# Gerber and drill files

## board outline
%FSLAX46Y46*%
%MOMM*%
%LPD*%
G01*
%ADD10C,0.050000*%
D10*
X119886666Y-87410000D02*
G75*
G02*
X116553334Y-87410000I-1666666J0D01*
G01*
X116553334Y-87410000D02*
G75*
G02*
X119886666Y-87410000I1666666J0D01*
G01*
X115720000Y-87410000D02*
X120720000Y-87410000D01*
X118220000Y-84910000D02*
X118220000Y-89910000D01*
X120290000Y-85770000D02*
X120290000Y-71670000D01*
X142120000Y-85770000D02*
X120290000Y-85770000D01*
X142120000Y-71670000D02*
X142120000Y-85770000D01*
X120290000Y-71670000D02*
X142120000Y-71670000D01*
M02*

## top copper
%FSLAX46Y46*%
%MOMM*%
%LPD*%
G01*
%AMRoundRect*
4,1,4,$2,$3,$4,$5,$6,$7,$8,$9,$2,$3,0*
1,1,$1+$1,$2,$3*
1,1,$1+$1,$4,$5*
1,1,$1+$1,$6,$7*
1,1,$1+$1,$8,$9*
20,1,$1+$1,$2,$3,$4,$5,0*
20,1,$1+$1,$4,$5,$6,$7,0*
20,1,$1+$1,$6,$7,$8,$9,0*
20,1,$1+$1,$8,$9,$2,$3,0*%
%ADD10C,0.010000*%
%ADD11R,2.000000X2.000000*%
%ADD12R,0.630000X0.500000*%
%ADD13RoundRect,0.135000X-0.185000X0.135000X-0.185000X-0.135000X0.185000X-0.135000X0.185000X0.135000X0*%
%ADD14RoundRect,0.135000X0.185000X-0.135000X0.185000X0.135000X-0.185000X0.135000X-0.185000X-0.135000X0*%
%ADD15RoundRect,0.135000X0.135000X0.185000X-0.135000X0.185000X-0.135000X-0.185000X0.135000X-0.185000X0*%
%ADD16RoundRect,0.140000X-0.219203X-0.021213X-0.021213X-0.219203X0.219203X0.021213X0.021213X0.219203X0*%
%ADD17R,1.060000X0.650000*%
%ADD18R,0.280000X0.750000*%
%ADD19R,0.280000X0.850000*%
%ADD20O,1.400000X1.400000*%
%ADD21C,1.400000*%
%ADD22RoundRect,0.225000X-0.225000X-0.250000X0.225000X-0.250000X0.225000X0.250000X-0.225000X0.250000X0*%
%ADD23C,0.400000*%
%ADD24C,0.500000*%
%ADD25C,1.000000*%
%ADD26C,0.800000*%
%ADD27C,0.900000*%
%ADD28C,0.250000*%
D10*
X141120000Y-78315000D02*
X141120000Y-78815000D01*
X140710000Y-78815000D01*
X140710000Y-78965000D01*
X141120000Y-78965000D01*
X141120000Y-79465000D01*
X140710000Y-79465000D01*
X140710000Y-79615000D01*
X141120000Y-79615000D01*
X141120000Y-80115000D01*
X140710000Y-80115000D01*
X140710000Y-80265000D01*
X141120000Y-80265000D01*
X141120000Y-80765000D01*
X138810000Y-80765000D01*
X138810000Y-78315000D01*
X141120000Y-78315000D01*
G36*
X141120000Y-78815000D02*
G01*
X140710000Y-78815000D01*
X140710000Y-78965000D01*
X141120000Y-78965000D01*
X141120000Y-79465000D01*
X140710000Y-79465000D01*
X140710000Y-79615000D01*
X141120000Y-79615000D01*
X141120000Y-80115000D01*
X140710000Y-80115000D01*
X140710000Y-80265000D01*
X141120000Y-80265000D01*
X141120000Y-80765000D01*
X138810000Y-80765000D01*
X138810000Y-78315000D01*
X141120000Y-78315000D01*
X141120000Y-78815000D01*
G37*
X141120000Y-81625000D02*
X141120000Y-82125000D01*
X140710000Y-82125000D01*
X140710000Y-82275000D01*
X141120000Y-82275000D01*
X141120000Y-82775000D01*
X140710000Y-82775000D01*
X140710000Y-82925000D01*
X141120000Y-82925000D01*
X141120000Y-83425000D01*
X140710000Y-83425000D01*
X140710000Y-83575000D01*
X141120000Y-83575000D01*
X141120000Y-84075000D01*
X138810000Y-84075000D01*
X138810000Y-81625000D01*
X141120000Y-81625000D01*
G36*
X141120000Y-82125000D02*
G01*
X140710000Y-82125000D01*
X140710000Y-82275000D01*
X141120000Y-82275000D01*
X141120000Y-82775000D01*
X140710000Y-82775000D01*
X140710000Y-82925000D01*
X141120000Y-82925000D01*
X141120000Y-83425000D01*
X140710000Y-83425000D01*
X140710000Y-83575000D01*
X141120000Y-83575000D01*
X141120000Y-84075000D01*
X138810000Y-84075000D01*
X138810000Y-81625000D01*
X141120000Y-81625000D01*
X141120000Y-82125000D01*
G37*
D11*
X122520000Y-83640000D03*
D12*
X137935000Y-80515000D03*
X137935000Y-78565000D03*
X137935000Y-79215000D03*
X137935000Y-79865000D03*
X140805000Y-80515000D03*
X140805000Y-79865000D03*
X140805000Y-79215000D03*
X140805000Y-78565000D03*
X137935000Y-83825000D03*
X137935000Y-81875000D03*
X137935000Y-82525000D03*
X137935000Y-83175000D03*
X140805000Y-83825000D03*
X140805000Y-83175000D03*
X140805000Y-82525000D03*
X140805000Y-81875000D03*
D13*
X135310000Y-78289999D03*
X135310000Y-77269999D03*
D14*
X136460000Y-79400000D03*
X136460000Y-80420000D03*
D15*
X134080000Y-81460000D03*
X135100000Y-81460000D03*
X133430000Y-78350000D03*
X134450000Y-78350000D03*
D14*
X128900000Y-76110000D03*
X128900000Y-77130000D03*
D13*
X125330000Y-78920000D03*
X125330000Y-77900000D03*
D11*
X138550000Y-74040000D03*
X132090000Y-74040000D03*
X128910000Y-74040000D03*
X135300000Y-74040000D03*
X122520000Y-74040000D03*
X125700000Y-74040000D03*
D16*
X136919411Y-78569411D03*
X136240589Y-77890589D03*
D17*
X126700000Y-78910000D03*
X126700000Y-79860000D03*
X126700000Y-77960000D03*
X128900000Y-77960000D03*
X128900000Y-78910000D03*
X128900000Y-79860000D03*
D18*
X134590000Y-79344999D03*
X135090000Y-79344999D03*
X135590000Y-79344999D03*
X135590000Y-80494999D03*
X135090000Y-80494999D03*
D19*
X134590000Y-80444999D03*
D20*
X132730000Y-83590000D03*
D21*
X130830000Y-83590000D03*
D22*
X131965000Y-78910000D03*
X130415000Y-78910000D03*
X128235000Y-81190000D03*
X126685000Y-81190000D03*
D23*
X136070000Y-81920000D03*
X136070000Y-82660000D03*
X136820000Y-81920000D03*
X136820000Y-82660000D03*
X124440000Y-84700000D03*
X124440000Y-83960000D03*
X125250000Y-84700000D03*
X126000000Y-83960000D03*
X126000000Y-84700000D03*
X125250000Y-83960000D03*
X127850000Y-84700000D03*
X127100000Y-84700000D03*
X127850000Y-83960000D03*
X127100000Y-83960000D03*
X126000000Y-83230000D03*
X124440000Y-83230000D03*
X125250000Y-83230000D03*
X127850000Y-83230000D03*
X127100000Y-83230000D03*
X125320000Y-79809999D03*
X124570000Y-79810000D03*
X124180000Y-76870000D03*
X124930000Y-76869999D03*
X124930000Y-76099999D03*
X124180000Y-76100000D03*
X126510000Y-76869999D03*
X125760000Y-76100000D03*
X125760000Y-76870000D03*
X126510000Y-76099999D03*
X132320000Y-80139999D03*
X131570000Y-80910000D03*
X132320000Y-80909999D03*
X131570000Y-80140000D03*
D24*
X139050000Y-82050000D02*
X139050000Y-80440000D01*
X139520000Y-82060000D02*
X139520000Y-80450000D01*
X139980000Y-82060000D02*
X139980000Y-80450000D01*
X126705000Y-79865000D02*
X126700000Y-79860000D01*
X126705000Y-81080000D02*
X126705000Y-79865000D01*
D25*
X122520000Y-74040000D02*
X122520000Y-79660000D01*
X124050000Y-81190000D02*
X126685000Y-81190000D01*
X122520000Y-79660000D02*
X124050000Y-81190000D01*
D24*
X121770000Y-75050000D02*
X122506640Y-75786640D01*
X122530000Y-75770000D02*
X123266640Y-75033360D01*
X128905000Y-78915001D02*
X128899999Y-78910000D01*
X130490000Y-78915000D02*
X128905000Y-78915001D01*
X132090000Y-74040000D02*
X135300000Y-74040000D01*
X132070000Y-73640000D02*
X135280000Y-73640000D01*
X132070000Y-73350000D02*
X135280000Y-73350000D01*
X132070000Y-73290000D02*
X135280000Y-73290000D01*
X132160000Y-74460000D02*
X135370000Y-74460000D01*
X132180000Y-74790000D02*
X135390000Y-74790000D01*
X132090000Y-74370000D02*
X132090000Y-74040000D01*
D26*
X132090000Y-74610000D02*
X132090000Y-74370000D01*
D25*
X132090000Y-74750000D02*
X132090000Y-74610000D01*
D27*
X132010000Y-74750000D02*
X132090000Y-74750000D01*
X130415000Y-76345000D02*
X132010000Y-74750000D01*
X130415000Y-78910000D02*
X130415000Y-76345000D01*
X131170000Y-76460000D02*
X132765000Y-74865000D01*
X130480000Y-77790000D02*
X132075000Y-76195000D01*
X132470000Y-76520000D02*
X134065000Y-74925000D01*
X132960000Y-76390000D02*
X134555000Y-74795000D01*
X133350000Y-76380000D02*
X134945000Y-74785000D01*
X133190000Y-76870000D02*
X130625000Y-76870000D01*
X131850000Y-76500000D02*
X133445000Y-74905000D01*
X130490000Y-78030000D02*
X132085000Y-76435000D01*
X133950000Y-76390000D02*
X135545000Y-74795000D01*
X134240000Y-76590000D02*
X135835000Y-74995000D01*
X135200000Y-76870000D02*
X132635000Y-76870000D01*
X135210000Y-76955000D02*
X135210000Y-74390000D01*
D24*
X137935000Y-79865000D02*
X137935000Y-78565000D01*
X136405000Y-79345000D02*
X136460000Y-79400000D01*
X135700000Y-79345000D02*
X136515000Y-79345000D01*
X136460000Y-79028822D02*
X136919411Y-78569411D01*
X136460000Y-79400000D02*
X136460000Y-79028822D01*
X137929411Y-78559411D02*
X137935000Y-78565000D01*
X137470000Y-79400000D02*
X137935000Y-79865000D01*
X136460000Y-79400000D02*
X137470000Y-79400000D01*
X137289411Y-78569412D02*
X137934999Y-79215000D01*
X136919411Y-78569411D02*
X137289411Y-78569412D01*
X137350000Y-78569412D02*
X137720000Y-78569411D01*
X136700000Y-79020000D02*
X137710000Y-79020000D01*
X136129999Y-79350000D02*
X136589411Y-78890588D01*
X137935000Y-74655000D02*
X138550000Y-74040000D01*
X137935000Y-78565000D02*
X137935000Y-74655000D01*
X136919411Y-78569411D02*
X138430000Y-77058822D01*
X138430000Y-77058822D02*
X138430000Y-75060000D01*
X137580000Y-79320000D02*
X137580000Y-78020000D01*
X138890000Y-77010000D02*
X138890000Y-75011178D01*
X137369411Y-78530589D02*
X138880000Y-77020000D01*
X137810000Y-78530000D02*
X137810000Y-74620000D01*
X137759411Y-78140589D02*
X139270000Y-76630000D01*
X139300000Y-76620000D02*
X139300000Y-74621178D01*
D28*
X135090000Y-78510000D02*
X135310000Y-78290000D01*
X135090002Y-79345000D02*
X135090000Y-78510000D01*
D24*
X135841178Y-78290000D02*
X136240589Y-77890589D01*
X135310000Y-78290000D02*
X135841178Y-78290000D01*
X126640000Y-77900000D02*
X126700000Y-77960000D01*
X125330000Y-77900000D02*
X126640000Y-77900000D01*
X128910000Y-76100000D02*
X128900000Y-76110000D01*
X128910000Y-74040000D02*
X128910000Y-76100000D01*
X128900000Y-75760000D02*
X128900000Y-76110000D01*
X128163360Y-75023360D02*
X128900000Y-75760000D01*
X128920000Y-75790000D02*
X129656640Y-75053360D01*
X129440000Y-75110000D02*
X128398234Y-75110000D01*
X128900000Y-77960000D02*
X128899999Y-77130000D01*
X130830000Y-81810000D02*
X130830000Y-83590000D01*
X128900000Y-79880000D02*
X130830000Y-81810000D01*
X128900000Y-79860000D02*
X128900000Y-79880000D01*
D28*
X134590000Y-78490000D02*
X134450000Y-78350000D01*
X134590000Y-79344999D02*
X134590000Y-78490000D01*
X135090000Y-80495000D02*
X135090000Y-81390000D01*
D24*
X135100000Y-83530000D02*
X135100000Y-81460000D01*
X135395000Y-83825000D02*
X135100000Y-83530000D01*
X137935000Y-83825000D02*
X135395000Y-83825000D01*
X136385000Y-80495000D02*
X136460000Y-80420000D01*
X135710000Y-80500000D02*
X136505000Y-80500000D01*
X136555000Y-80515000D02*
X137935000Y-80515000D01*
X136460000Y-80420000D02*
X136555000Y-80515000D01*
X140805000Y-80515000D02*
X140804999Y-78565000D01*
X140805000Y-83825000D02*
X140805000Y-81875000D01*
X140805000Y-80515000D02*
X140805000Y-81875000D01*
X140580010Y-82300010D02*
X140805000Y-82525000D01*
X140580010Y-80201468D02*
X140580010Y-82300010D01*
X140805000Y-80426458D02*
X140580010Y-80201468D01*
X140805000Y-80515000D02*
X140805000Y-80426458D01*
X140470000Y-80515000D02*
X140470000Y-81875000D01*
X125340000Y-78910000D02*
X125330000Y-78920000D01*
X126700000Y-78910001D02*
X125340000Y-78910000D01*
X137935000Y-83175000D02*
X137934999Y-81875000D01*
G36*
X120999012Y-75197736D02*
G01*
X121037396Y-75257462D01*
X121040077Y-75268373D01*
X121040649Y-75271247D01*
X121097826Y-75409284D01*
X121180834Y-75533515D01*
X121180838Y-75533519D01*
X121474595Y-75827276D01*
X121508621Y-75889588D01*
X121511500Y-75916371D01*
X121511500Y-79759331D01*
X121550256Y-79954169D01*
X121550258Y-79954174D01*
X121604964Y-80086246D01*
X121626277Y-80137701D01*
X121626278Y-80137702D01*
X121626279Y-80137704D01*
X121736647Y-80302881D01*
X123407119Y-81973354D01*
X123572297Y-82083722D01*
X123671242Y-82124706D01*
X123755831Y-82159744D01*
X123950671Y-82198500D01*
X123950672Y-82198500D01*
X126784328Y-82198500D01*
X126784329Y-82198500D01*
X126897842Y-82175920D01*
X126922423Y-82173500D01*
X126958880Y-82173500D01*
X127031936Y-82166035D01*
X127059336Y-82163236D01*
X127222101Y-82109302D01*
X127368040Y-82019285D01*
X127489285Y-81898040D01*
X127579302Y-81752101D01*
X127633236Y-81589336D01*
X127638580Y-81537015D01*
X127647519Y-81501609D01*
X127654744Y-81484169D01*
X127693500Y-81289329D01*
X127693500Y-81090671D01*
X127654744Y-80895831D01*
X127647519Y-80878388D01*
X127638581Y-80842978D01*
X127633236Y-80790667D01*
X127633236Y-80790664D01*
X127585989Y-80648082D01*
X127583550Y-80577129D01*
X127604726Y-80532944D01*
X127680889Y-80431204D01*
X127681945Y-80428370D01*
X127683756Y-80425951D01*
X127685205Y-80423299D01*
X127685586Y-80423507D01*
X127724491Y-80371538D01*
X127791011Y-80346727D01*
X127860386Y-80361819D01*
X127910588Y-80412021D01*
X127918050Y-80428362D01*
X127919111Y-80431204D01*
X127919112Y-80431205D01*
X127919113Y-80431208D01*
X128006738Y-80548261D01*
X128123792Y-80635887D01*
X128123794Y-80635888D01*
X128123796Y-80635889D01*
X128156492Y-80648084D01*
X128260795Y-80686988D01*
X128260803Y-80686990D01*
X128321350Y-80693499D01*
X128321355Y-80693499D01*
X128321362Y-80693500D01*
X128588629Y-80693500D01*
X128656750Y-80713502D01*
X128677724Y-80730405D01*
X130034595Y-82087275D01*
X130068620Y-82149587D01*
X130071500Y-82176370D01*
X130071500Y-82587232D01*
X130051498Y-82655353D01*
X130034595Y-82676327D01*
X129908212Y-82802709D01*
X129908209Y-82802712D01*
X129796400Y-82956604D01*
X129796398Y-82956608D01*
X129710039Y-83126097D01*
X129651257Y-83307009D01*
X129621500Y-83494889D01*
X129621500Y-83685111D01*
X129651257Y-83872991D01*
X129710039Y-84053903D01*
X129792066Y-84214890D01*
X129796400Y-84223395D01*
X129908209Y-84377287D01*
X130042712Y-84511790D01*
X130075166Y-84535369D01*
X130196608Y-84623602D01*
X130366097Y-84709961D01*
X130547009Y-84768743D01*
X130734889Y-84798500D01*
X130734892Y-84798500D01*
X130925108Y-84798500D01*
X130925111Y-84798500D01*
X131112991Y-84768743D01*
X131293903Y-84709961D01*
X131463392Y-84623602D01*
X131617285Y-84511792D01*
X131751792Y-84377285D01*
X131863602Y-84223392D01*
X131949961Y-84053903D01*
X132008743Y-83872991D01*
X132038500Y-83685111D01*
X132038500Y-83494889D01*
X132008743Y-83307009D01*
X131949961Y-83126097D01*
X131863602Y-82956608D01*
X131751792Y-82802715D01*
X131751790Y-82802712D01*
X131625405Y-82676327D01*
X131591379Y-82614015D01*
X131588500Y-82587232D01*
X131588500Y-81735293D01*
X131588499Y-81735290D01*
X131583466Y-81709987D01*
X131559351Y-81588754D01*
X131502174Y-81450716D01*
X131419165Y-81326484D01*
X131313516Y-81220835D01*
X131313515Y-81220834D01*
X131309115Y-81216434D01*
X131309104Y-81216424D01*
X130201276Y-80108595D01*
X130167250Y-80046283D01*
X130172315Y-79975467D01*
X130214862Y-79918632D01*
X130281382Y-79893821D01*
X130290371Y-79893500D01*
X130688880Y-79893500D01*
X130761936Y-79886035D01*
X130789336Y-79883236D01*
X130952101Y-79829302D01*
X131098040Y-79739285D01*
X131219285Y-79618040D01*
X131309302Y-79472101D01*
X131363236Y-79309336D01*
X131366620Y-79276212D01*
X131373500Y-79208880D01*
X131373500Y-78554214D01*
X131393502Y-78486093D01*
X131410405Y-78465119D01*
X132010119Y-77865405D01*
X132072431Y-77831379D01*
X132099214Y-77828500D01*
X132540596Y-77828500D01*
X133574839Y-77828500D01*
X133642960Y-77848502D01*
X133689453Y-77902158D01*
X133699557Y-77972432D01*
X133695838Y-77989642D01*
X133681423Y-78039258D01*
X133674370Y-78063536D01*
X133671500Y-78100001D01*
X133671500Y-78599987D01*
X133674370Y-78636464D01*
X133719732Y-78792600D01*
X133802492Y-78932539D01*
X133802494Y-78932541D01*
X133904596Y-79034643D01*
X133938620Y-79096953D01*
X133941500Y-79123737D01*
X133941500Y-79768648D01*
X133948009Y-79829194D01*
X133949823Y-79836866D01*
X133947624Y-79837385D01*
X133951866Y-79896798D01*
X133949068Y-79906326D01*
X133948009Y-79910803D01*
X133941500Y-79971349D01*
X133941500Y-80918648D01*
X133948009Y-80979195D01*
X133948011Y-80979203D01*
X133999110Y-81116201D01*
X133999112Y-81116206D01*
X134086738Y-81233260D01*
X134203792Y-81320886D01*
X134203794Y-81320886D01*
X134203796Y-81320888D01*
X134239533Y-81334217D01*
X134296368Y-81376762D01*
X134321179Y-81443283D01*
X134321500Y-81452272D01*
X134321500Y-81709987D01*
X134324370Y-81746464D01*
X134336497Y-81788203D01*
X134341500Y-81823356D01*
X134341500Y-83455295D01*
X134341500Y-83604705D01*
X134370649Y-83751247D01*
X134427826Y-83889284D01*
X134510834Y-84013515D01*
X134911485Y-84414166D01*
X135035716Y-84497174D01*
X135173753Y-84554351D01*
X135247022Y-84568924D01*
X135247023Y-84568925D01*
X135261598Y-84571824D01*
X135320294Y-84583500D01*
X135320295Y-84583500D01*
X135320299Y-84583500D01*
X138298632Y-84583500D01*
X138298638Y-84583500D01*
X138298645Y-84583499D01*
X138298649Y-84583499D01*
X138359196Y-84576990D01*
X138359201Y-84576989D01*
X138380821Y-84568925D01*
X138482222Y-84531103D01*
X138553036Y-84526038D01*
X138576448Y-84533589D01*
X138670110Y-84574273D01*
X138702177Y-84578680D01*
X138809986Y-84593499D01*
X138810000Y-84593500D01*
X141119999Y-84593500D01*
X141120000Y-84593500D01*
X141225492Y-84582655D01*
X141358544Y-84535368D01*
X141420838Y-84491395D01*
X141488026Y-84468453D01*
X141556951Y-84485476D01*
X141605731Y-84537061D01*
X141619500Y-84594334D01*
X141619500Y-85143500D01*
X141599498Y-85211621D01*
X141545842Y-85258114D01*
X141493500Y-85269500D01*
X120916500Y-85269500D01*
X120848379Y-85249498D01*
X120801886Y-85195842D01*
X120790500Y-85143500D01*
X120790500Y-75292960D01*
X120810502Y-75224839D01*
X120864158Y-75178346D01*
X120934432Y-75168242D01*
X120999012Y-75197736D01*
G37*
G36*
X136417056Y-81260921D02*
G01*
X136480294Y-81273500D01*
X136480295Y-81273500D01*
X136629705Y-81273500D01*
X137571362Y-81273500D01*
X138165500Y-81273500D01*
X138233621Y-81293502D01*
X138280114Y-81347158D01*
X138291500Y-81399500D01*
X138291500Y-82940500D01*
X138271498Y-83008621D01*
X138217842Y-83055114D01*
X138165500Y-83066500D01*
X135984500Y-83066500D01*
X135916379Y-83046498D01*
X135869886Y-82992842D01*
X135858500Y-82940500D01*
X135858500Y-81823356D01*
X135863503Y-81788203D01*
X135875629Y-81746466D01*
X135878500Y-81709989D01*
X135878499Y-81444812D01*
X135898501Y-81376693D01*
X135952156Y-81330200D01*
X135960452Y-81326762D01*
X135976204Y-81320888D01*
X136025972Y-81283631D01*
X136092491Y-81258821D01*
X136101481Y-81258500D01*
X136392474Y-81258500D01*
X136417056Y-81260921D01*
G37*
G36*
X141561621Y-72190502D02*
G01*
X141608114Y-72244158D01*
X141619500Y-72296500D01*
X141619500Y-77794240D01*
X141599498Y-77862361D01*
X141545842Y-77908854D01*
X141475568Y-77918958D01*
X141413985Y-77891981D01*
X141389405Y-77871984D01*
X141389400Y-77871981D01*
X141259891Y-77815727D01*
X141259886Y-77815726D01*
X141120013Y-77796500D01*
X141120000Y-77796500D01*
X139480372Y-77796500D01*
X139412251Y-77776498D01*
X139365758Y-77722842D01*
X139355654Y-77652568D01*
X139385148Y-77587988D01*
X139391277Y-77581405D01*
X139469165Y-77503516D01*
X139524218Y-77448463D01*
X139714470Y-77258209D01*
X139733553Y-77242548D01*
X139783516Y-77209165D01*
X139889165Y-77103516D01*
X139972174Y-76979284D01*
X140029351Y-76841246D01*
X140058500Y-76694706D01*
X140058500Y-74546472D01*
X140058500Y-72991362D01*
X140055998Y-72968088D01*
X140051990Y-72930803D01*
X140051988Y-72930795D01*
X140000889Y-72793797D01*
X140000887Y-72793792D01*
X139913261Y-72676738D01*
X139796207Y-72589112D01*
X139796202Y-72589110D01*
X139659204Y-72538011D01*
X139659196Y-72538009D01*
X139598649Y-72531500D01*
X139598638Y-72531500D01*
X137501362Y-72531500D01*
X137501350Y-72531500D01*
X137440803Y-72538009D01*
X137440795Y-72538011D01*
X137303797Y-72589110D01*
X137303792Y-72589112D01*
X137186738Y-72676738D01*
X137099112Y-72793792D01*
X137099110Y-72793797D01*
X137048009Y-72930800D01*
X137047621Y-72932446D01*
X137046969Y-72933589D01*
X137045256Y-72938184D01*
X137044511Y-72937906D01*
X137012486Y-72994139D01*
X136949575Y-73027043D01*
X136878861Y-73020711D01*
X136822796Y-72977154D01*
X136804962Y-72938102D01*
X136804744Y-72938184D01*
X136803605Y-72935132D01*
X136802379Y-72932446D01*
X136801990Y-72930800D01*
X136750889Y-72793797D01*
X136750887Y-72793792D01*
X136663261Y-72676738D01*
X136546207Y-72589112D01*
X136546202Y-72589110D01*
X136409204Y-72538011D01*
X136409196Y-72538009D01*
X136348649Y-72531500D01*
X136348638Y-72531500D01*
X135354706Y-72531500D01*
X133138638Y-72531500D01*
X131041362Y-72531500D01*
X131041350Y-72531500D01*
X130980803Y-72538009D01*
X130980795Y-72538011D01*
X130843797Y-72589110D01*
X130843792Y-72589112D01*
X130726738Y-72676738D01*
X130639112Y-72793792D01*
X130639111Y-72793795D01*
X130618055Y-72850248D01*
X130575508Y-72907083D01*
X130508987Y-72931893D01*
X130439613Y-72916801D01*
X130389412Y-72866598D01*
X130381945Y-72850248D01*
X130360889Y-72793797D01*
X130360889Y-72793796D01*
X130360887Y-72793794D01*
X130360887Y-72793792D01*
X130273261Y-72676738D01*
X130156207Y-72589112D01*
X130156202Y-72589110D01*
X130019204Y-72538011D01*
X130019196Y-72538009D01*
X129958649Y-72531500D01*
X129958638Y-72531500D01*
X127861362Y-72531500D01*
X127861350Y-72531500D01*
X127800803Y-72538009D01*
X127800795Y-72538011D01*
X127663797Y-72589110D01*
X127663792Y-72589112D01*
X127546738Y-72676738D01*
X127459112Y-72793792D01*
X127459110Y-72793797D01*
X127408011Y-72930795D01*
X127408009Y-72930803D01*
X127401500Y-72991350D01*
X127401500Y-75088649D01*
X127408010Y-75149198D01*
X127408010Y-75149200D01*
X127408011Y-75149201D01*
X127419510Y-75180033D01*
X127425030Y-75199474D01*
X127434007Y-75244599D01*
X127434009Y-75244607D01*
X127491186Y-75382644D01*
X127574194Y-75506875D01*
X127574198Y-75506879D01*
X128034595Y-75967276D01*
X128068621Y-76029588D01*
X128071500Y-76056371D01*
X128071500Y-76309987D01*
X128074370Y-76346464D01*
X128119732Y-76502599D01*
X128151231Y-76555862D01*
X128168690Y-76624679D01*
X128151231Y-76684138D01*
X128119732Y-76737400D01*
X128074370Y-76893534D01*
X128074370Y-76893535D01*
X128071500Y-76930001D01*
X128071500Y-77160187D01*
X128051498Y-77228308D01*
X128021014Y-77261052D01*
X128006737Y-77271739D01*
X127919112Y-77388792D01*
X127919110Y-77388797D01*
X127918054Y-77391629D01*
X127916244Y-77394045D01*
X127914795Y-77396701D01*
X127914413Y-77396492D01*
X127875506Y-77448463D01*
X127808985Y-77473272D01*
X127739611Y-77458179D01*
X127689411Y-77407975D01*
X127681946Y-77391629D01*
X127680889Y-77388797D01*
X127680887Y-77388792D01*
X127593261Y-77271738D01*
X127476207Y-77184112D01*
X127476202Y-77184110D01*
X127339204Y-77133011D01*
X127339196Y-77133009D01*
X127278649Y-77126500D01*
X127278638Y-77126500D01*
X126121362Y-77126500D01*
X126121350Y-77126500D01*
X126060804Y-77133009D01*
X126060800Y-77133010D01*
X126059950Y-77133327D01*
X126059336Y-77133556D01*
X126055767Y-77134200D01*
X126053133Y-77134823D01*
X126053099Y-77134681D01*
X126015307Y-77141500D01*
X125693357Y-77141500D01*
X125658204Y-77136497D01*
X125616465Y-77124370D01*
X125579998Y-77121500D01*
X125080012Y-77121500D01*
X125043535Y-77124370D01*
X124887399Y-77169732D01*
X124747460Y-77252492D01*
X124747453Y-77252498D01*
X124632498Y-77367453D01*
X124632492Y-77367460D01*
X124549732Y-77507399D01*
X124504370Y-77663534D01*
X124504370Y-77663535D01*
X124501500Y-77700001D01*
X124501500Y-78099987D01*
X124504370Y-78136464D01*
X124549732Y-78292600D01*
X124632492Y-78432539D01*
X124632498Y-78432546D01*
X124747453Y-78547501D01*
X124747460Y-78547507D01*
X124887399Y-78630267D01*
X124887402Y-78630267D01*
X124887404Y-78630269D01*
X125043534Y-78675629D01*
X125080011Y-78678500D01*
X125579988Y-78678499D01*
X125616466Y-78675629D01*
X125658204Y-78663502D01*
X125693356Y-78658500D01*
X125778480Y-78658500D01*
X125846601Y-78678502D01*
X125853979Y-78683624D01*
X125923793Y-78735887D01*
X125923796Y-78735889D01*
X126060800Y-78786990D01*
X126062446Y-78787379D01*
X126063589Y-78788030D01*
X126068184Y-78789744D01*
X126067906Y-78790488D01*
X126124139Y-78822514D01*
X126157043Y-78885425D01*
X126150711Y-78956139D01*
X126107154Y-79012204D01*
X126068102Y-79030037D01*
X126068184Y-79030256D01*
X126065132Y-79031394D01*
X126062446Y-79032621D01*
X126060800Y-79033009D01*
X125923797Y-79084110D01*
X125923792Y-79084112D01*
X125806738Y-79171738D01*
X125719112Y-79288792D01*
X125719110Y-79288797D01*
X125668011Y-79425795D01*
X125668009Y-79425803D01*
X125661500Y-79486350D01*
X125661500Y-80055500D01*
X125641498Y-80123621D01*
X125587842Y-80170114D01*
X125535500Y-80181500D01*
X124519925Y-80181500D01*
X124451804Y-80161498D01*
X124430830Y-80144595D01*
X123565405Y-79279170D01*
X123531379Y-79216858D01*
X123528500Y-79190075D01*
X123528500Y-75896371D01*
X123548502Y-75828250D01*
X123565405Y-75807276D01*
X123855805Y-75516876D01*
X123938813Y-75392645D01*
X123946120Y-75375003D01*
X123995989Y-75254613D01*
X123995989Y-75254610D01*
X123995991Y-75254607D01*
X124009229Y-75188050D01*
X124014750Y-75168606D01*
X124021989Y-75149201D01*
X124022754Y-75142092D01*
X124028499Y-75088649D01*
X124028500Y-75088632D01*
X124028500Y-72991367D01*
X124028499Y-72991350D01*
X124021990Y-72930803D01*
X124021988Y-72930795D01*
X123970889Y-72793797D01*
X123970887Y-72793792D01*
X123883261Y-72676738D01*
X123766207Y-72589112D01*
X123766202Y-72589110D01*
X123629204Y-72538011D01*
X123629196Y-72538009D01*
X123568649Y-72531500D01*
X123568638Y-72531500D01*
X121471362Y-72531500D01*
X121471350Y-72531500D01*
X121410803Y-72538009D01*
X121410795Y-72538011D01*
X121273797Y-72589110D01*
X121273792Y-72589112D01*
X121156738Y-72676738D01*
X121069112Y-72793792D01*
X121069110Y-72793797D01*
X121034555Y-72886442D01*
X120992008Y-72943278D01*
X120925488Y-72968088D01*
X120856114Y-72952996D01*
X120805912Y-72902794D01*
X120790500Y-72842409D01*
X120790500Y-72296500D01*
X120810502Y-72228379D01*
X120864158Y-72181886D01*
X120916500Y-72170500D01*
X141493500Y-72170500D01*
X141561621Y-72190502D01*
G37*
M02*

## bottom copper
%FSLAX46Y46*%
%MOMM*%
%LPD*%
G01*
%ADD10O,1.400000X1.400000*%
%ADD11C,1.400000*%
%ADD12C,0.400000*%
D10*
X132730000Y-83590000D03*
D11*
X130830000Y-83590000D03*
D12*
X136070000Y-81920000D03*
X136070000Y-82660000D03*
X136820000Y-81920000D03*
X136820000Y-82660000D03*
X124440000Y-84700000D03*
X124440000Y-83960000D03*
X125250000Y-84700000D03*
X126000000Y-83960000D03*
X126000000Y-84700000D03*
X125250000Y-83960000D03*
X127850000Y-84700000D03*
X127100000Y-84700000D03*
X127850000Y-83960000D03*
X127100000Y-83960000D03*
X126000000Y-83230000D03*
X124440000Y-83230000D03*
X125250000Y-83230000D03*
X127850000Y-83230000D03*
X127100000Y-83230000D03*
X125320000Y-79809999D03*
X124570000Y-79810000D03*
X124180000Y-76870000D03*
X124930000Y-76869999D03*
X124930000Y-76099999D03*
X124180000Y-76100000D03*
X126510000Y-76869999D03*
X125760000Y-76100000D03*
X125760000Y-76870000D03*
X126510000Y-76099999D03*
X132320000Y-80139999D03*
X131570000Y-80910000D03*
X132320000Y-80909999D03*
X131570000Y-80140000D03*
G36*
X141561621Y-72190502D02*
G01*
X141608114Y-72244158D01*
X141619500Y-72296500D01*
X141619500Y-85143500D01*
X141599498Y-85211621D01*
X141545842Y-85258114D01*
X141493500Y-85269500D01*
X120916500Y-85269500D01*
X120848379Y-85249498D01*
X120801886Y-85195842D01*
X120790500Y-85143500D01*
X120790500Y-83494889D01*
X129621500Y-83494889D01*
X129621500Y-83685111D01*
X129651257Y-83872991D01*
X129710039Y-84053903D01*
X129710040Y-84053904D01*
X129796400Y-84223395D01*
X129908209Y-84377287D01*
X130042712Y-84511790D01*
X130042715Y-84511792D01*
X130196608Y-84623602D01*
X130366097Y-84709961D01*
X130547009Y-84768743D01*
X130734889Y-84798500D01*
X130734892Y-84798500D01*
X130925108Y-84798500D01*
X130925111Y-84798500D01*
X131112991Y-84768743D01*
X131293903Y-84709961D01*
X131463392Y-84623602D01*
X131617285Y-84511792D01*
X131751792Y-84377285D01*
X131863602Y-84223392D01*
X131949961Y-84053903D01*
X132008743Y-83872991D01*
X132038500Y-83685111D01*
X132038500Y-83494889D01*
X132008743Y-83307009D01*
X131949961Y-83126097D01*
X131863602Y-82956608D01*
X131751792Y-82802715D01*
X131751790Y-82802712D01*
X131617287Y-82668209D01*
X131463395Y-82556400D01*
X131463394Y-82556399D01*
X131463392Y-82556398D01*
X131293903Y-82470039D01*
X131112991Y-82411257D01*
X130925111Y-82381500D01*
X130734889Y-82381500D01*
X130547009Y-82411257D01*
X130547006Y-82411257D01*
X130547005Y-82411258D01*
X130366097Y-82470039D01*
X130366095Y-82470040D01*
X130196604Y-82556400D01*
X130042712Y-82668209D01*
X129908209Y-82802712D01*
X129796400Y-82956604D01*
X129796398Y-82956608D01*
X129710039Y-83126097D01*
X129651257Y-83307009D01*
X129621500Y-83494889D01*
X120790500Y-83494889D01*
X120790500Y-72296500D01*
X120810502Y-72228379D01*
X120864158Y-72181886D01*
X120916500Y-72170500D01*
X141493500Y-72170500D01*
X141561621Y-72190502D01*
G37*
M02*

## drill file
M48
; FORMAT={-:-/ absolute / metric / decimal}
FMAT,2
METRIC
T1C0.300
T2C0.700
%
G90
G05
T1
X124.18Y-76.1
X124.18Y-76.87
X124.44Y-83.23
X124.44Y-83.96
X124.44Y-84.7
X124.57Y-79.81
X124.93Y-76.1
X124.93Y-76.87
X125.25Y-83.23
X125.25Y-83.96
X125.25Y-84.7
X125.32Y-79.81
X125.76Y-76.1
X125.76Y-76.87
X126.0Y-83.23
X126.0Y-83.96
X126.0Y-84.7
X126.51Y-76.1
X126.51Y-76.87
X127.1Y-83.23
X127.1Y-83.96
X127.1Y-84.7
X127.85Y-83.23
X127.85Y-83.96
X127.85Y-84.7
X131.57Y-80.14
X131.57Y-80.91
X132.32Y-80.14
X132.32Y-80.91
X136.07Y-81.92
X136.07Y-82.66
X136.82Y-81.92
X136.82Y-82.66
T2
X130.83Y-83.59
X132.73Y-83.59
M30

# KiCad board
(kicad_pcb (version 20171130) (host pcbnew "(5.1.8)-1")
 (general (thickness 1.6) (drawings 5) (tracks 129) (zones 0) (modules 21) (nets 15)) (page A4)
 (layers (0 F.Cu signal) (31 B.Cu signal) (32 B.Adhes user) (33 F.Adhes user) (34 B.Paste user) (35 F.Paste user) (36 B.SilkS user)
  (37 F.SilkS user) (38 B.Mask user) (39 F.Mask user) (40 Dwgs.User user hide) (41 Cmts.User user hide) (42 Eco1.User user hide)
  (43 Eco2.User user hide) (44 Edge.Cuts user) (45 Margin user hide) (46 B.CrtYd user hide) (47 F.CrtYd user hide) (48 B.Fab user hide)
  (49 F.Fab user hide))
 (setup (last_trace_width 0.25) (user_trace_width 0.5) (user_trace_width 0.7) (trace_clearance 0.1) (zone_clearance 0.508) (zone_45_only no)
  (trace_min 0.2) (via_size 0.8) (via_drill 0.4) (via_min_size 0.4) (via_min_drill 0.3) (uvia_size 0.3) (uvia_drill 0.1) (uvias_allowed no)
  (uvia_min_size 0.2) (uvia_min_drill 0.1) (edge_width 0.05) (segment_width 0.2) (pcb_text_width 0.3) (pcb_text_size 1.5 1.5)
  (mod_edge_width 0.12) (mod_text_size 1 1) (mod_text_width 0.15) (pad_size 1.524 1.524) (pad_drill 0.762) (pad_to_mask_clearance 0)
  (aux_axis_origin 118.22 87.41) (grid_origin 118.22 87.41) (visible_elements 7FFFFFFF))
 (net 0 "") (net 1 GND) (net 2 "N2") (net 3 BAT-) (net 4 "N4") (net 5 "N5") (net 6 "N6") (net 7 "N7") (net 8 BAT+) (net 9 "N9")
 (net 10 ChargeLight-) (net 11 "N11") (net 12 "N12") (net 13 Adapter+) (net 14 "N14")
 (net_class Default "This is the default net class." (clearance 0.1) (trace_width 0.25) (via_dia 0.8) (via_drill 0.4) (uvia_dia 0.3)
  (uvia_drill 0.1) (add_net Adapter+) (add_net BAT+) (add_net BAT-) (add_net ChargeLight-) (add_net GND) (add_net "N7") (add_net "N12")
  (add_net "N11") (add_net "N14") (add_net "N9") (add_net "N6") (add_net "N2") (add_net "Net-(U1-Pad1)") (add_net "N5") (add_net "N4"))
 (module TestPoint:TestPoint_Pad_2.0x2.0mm (layer F.Cu) (at 122.52 83.64)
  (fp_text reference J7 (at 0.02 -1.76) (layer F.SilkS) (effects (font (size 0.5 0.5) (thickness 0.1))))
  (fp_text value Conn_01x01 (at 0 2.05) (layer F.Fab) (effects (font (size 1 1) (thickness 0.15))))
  (pad 1 smd rect (at 0 0) (size 2 2) (layers F.Cu F.Mask) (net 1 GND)))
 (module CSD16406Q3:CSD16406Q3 (layer F.Cu) (at 139.37 79.54)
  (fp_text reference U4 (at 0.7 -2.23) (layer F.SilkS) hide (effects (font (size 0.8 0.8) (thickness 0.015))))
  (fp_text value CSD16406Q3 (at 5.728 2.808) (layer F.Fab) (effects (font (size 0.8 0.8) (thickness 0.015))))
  (fp_poly
   (pts (xy 1.75 -1.225) (xy 1.75 -0.725) (xy 1.34 -0.725) (xy 1.34 -0.575) (xy 1.75 -0.575) (xy 1.75 -0.075) (xy 1.34 -0.075)
    (xy 1.34 0.075) (xy 1.75 0.075) (xy 1.75 0.575) (xy 1.34 0.575) (xy 1.34 0.725) (xy 1.75 0.725) (xy 1.75 1.225) (xy -0.56 1.225)
    (xy -0.56 -1.225))
   (layer F.Cu) (width 0.01))
  (pad 4 smd rect (at -1.435 0.975) (size 0.63 0.5) (layers F.Cu F.Mask) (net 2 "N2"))
  (pad 1 smd rect (at -1.435 -0.975) (size 0.63 0.5) (layers F.Cu F.Mask) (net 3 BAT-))
  (pad 2 smd rect (at -1.435 -0.325) (size 0.63 0.5) (layers F.Cu F.Mask) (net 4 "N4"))
  (pad 3 smd rect (at -1.435 0.325) (size 0.63 0.5) (layers F.Cu F.Mask) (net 4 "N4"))
  (pad 5 smd rect (at 1.435 0.975) (size 0.63 0.5) (layers F.Cu) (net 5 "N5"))
  (pad 6 smd rect (at 1.435 0.325) (size 0.63 0.5) (layers F.Cu) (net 5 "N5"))
  (pad 7 smd rect (at 1.435 -0.325) (size 0.63 0.5) (layers F.Cu) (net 5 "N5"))
  (pad 8 smd rect (at 1.435 -0.975) (size 0.63 0.5) (layers F.Cu) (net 5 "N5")))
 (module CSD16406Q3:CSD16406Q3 (layer F.Cu) (at 139.37 82.85)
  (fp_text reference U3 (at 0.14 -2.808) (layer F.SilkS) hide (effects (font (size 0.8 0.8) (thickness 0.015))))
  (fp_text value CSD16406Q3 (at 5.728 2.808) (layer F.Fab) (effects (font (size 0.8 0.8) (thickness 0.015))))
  (fp_poly
   (pts (xy 1.75 -1.225) (xy 1.75 -0.725) (xy 1.34 -0.725) (xy 1.34 -0.575) (xy 1.75 -0.575) (xy 1.75 -0.075) (xy 1.34 -0.075)
    (xy 1.34 0.075) (xy 1.75 0.075) (xy 1.75 0.575) (xy 1.34 0.575) (xy 1.34 0.725) (xy 1.75 0.725) (xy 1.75 1.225) (xy -0.56 1.225)
    (xy -0.56 -1.225))
   (layer F.Cu) (width 0.01))
  (pad 4 smd rect (at -1.435 0.975) (size 0.63 0.5) (layers F.Cu F.Mask) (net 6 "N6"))
  (pad 1 smd rect (at -1.435 -0.975) (size 0.63 0.5) (layers F.Cu F.Mask) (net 1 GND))
  (pad 2 smd rect (at -1.435 -0.325) (size 0.63 0.5) (layers F.Cu F.Mask) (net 1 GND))
  (pad 3 smd rect (at -1.435 0.325) (size 0.63 0.5) (layers F.Cu F.Mask) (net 1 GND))
  (pad 5 smd rect (at 1.435 0.975) (size 0.63 0.5) (layers F.Cu) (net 5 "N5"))
  (pad 6 smd rect (at 1.435 0.325) (size 0.63 0.5) (layers F.Cu) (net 5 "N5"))
  (pad 7 smd rect (at 1.435 -0.325) (size 0.63 0.5) (layers F.Cu) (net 5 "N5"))
  (pad 8 smd rect (at 1.435 -0.975) (size 0.63 0.5) (layers F.Cu) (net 5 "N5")))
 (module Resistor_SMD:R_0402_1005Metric (layer F.Cu) (at 135.31 77.779999 270)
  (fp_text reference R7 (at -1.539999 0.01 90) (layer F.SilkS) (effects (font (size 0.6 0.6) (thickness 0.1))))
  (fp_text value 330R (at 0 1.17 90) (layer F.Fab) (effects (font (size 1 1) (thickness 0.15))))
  (pad 2 smd roundrect (at 0.51 0 270) (size 0.54 0.64) (layers F.Cu F.Paste F.Mask) (roundrect_rratio 0.25) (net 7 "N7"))
  (pad 1 smd roundrect (at -0.51 0 270) (size 0.54 0.64) (layers F.Cu F.Paste F.Mask) (roundrect_rratio 0.25) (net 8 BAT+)))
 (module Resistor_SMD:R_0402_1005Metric (layer F.Cu) (at 136.46 79.91 90)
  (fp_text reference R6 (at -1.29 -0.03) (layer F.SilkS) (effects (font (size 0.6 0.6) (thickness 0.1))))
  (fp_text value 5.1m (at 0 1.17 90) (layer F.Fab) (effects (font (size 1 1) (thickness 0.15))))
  (pad 2 smd roundrect (at 0.51 0 90) (size 0.54 0.64) (layers F.Cu F.Paste F.Mask) (roundrect_rratio 0.25) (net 3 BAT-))
  (pad 1 smd roundrect (at -0.51 0 90) (size 0.54 0.64) (layers F.Cu F.Paste F.Mask) (roundrect_rratio 0.25) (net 2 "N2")))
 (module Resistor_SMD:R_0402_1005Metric (layer F.Cu) (at 134.59 81.46 180)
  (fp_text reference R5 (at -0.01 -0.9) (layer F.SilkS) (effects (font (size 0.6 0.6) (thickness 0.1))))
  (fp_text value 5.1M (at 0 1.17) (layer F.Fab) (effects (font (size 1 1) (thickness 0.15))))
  (pad 2 smd roundrect (at 0.51 0 180) (size 0.54 0.64) (layers F.Cu F.Paste F.Mask) (roundrect_rratio 0.25) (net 1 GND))
  (pad 1 smd roundrect (at -0.51 0 180) (size 0.54 0.64) (layers F.Cu F.Paste F.Mask) (roundrect_rratio 0.25) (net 6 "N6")))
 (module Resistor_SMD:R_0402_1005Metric (layer F.Cu) (at 133.94 78.35 180)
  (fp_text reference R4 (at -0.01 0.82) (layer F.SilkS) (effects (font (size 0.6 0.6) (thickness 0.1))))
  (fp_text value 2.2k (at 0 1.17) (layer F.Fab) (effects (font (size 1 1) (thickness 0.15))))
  (pad 2 smd roundrect (at 0.51 0 180) (size 0.54 0.64) (layers F.Cu F.Paste F.Mask) (roundrect_rratio 0.25) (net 1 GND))
  (pad 1 smd roundrect (at -0.51 0 180) (size 0.54 0.64) (layers F.Cu F.Paste F.Mask) (roundrect_rratio 0.25) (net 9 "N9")))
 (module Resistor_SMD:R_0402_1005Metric (layer F.Cu) (at 128.9 76.62 90)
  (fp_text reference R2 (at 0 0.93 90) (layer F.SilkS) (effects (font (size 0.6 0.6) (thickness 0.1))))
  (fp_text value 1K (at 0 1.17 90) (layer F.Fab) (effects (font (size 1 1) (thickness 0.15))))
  (pad 2 smd roundrect (at 0.51 0 90) (size 0.54 0.64) (layers F.Cu F.Paste F.Mask) (roundrect_rratio 0.25) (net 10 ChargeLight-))
  (pad 1 smd roundrect (at -0.51 0 90) (size 0.54 0.64) (layers F.Cu F.Paste F.Mask) (roundrect_rratio 0.25) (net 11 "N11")))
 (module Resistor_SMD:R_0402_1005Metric (layer F.Cu) (at 125.33 78.41 270)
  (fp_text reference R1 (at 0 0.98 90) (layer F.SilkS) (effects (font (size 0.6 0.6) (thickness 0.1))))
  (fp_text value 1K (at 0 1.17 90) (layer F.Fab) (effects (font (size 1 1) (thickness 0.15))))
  (pad 2 smd roundrect (at 0.51 0 270) (size 0.54 0.64) (layers F.Cu F.Paste F.Mask) (roundrect_rratio 0.25) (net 1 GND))
  (pad 1 smd roundrect (at -0.51 0 270) (size 0.54 0.64) (layers F.Cu F.Paste F.Mask) (roundrect_rratio 0.25) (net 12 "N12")))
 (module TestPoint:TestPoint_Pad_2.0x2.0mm (layer F.Cu) (at 138.55 74.04 180)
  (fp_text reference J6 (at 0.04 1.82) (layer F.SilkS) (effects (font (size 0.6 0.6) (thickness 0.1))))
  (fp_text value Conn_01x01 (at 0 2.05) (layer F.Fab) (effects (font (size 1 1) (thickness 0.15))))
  (pad 1 smd rect (at 0 0 180) (size 2 2) (layers F.Cu F.Mask) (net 3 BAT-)))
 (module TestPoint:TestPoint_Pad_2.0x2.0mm (layer F.Cu) (at 132.09 74.04 180)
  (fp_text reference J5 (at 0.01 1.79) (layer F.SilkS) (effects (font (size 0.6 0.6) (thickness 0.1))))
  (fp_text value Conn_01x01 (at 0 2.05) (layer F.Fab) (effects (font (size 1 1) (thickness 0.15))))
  (pad 1 smd rect (at 0 0 180) (size 2 2) (layers F.Cu F.Mask) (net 8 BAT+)))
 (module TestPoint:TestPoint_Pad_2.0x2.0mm (layer F.Cu) (at 128.91 74.04 180)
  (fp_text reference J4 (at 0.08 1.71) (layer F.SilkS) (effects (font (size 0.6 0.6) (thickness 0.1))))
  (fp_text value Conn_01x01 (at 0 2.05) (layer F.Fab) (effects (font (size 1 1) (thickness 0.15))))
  (pad 1 smd rect (at 0 0 180) (size 2 2) (layers F.Cu F.Mask) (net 10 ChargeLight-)))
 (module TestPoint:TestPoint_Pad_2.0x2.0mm (layer F.Cu) (at 135.3 74.04 180)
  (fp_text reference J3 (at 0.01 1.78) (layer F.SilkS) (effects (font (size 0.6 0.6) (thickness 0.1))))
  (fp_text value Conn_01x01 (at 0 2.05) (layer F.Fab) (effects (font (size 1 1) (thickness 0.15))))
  (pad 1 smd rect (at 0 0 180) (size 2 2) (layers F.Cu F.Mask) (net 8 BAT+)))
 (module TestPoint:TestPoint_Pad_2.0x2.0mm (layer F.Cu) (at 122.52 74.04 180)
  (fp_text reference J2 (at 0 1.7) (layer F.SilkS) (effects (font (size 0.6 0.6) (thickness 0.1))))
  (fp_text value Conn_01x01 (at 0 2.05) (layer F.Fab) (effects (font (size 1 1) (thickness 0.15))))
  (pad 1 smd rect (at 0 0 180) (size 2 2) (layers F.Cu F.Mask) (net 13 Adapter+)))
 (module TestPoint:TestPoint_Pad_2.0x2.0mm (layer F.Cu) (at 125.7 74.04 180)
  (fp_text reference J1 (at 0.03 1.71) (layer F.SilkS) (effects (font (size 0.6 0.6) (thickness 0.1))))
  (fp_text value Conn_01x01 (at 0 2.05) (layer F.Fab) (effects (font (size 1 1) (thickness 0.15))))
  (pad 1 smd rect (at 0 0 180) (size 2 2) (layers F.Cu F.Mask) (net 1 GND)))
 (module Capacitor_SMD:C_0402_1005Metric (layer F.Cu) (at 136.58 78.23 315)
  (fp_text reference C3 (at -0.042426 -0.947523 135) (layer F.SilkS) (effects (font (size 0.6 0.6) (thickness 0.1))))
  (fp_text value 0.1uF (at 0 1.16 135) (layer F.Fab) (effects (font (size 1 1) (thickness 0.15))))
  (pad 2 smd roundrect (at 0.48 0 315) (size 0.56 0.62) (layers F.Cu F.Paste F.Mask) (roundrect_rratio 0.25) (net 3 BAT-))
  (pad 1 smd roundrect (at -0.48 0 315) (size 0.56 0.62) (layers F.Cu F.Paste F.Mask) (roundrect_rratio 0.25) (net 7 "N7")))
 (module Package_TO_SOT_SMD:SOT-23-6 (layer F.Cu) (at 127.8 78.91 180)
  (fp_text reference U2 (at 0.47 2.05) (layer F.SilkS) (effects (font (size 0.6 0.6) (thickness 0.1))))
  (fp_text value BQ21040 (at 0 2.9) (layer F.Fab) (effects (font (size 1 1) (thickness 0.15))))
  (pad 5 smd rect (at 1.1 0 180) (size 1.06 0.65) (layers F.Cu F.Paste F.Mask) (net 1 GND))
  (pad 6 smd rect (at 1.1 -0.95 180) (size 1.06 0.65) (layers F.Cu F.Paste F.Mask) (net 13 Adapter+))
  (pad 4 smd rect (at 1.1 0.95 180) (size 1.06 0.65) (layers F.Cu F.Paste F.Mask) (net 12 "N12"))
  (pad 3 smd rect (at -1.1 0.95 180) (size 1.06 0.65) (layers F.Cu F.Paste F.Mask) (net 11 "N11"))
  (pad 2 smd rect (at -1.1 0 180) (size 1.06 0.65) (layers F.Cu F.Paste F.Mask) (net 8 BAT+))
  (pad 1 smd rect (at -1.1 -0.95 180) (size 1.06 0.65) (layers F.Cu F.Paste F.Mask) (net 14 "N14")))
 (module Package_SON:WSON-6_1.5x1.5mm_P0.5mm (layer F.Cu) (at 135.09 79.919999 90)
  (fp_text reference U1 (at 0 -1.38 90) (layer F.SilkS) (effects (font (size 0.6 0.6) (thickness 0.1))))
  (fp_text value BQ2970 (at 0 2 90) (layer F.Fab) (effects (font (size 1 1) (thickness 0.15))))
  (pad 6 smd rect (at 0.575 -0.5) (size 0.28 0.75) (layers F.Cu F.Paste F.Mask) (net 9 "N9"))
  (pad 5 smd rect (at 0.575 0) (size 0.28 0.75) (layers F.Cu F.Paste F.Mask) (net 7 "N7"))
  (pad 4 smd rect (at 0.575 0.5) (size 0.28 0.75) (layers F.Cu F.Paste F.Mask) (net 3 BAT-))
  (pad 3 smd rect (at -0.575 0.5) (size 0.28 0.75) (layers F.Cu F.Paste F.Mask) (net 2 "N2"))
  (pad 2 smd rect (at -0.575 0) (size 0.28 0.75) (layers F.Cu F.Paste F.Mask) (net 6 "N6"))
  (pad 1 smd rect (at -0.525 -0.5) (size 0.28 0.85) (layers F.Cu F.Paste F.Mask)))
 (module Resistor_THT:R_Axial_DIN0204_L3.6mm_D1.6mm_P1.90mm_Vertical (layer F.Cu) (at 130.83 83.59)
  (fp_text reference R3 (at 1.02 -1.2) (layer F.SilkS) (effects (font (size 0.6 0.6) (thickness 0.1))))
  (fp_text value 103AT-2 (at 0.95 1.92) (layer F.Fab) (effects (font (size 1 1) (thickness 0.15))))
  (pad 2 thru_hole oval (at 1.9 0) (size 1.4 1.4) (drill 0.7) (layers *.Cu *.Mask) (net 1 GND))
  (pad 1 thru_hole circle (at 0 0) (size 1.4 1.4) (drill 0.7) (layers *.Cu *.Mask) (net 14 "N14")))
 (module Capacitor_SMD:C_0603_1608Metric (layer F.Cu) (at 131.19 78.91)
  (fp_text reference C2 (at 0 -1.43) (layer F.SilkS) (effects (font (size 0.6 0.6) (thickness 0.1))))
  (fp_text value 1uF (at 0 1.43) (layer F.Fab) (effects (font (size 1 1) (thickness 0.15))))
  (pad 2 smd roundrect (at 0.775 0) (size 0.9 0.95) (layers F.Cu F.Paste F.Mask) (roundrect_rratio 0.25) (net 1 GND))
  (pad 1 smd roundrect (at -0.775 0) (size 0.9 0.95) (layers F.Cu F.Paste F.Mask) (roundrect_rratio 0.25) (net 8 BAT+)))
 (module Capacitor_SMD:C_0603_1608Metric (layer F.Cu) (at 127.46 81.19)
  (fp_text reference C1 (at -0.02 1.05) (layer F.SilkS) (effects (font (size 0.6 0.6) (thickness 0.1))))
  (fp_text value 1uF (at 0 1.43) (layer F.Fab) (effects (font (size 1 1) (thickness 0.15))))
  (pad 2 smd roundrect (at 0.775 0) (size 0.9 0.95) (layers F.Cu F.Paste F.Mask) (roundrect_rratio 0.25) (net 1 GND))
  (pad 1 smd roundrect (at -0.775 0) (size 0.9 0.95) (layers F.Cu F.Paste F.Mask) (roundrect_rratio 0.25) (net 13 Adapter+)))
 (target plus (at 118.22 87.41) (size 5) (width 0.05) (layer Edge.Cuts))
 (gr_line (start 120.29 85.77) (end 120.29 71.67) (layer Edge.Cuts) (width 0.05))
 (gr_line (start 142.12 85.77) (end 120.29 85.77) (layer Edge.Cuts) (width 0.05))
 (gr_line (start 142.12 71.67) (end 142.12 85.77) (layer Edge.Cuts) (width 0.05))
 (gr_line (start 120.29 71.67) (end 142.12 71.67) (layer Edge.Cuts) (width 0.05))
 (segment (start 139.05 82.05) (end 139.05 80.44) (width 0.5) (layer F.Cu) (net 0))
 (segment (start 139.52 82.06) (end 139.52 80.45) (width 0.5) (layer F.Cu) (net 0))
 (segment (start 139.98 82.06) (end 139.98 80.45) (width 0.5) (layer F.Cu) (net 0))
 (segment (start 126.705 79.865) (end 126.7 79.86) (width 0.5) (layer F.Cu) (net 13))
 (segment (start 126.705 81.08) (end 126.705 79.865) (width 0.5) (layer F.Cu) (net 13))
 (segment (start 122.52 74.04) (end 122.52 79.66) (width 1) (layer F.Cu) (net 13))
 (segment (start 124.05 81.19) (end 126.685 81.19) (width 1) (layer F.Cu) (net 13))
 (segment (start 122.52 79.66) (end 124.05 81.19) (width 1) (layer F.Cu) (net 13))
 (segment (start 121.77 75.05) (end 122.50664 75.78664) (width 0.5) (layer F.Cu) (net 13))
 (segment (start 122.53 75.77) (end 123.26664 75.03336) (width 0.5) (layer F.Cu) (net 13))
 (segment (start 128.905 78.915001) (end 128.899999 78.91) (width 0.5) (layer F.Cu) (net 8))
 (segment (start 130.49 78.915) (end 128.905 78.915001) (width 0.5) (layer F.Cu) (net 8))
 (segment (start 132.09 74.04) (end 135.3 74.04) (width 0.5) (layer F.Cu) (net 8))
 (segment (start 132.07 73.64) (end 135.28 73.64) (width 0.5) (layer F.Cu) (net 8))
 (segment (start 132.07 73.35) (end 135.28 73.35) (width 0.5) (layer F.Cu) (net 8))
 (segment (start 132.07 73.29) (end 135.28 73.29) (width 0.5) (layer F.Cu) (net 8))
 (segment (start 132.16 74.46) (end 135.37 74.46) (width 0.5) (layer F.Cu) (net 8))
 (segment (start 132.18 74.79) (end 135.39 74.79) (width 0.5) (layer F.Cu) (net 8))
 (segment (start 132.09 74.37) (end 132.09 74.04) (width 0.5) (layer F.Cu) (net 8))
 (segment (start 132.09 74.61) (end 132.09 74.37) (width 0.8) (layer F.Cu) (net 8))
 (segment (start 132.09 74.75) (end 132.09 74.61) (width 1) (layer F.Cu) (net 8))
 (segment (start 132.01 74.75) (end 132.09 74.75) (width 0.9) (layer F.Cu) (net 8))
 (segment (start 130.415 76.345) (end 132.01 74.75) (width 0.9) (layer F.Cu) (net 8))
 (segment (start 130.415 78.91) (end 130.415 76.345) (width 0.9) (layer F.Cu) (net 8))
 (segment (start 131.17 76.46) (end 132.765 74.865) (width 0.9) (layer F.Cu) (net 8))
 (segment (start 130.48 77.79) (end 132.075 76.195) (width 0.9) (layer F.Cu) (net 8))
 (segment (start 132.47 76.52) (end 134.065 74.925) (width 0.9) (layer F.Cu) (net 8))
 (segment (start 132.96 76.39) (end 134.555 74.795) (width 0.9) (layer F.Cu) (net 8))
 (segment (start 133.35 76.38) (end 134.945 74.785) (width 0.9) (layer F.Cu) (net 8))
 (segment (start 133.19 76.87) (end 130.625 76.87) (width 0.9) (layer F.Cu) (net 8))
 (segment (start 131.85 76.5) (end 133.445 74.905) (width 0.9) (layer F.Cu) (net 8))
 (segment (start 130.49 78.03) (end 132.085 76.435) (width 0.9) (layer F.Cu) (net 8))
 (segment (start 133.95 76.39) (end 135.545 74.795) (width 0.9) (layer F.Cu) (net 8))
 (segment (start 134.24 76.59) (end 135.835 74.995) (width 0.9) (layer F.Cu) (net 8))
 (segment (start 135.2 76.87) (end 132.635 76.87) (width 0.9) (layer F.Cu) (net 8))
 (segment (start 135.21 76.955) (end 135.21 74.39) (width 0.9) (layer F.Cu) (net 8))
 (segment (start 137.935 79.865) (end 137.935 78.565) (width 0.5) (layer F.Cu) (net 3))
 (segment (start 136.405 79.345) (end 136.46 79.4) (width 0.5) (layer F.Cu) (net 3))
 (segment (start 135.7 79.345) (end 136.515 79.345) (width 0.5) (layer F.Cu) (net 3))
 (segment (start 136.46 79.028822) (end 136.919411 78.569411) (width 0.5) (layer F.Cu) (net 3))
 (segment (start 136.46 79.4) (end 136.46 79.028822) (width 0.5) (layer F.Cu) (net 3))
 (segment (start 137.929411 78.559411) (end 137.935 78.565) (width 0.5) (layer F.Cu) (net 3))
 (segment (start 137.47 79.4) (end 137.935 79.865) (width 0.5) (layer F.Cu) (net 3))
 (segment (start 136.46 79.4) (end 137.47 79.4) (width 0.5) (layer F.Cu) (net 3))
 (segment (start 137.289411 78.569412) (end 137.934999 79.215) (width 0.5) (layer F.Cu) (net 3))
 (segment (start 136.919411 78.569411) (end 137.289411 78.569412) (width 0.5) (layer F.Cu) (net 3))
 (segment (start 137.35 78.569412) (end 137.72 78.569411) (width 0.5) (layer F.Cu) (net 3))
 (segment (start 136.7 79.02) (end 137.71 79.02) (width 0.5) (layer F.Cu) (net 3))
 (segment (start 136.129999 79.35) (end 136.589411 78.890588) (width 0.5) (layer F.Cu) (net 3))
 (segment (start 137.935 74.655) (end 138.55 74.04) (width 0.5) (layer F.Cu) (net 3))
 (segment (start 137.935 78.565) (end 137.935 74.655) (width 0.5) (layer F.Cu) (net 3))
 (segment (start 136.919411 78.569411) (end 138.43 77.058822) (width 0.5) (layer F.Cu) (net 3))
 (segment (start 138.43 77.058822) (end 138.43 75.06) (width 0.5) (layer F.Cu) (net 3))
 (segment (start 137.58 79.32) (end 137.58 78.02) (width 0.5) (layer F.Cu) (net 3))
 (segment (start 138.89 77.01) (end 138.89 75.011178) (width 0.5) (layer F.Cu) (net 3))
 (segment (start 137.369411 78.530589) (end 138.88 77.02) (width 0.5) (layer F.Cu) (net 3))
 (segment (start 137.81 78.53) (end 137.81 74.62) (width 0.5) (layer F.Cu) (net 3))
 (segment (start 137.759411 78.140589) (end 139.27 76.63) (width 0.5) (layer F.Cu) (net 3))
 (segment (start 139.3 76.62) (end 139.3 74.621178) (width 0.5) (layer F.Cu) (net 3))
 (segment (start 135.09 78.51) (end 135.31 78.29) (width 0.25) (layer F.Cu) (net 7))
 (segment (start 135.090002 79.345) (end 135.09 78.51) (width 0.25) (layer F.Cu) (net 7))
 (segment (start 135.841178 78.29) (end 136.240589 77.890589) (width 0.5) (layer F.Cu) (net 7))
 (segment (start 135.31 78.29) (end 135.841178 78.29) (width 0.5) (layer F.Cu) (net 7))
 (segment (start 126.64 77.9) (end 126.7 77.96) (width 0.5) (layer F.Cu) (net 12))
 (segment (start 125.33 77.9) (end 126.64 77.9) (width 0.5) (layer F.Cu) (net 12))
 (segment (start 128.91 76.1) (end 128.9 76.11) (width 0.5) (layer F.Cu) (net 10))
 (segment (start 128.91 74.04) (end 128.91 76.1) (width 0.5) (layer F.Cu) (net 10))
 (segment (start 128.9 75.76) (end 128.9 76.11) (width 0.5) (layer F.Cu) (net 10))
 (segment (start 128.16336 75.02336) (end 128.9 75.76) (width 0.5) (layer F.Cu) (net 10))
 (segment (start 128.92 75.79) (end 129.65664 75.05336) (width 0.5) (layer F.Cu) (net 10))
 (segment (start 129.44 75.11) (end 128.398234 75.11) (width 0.5) (layer F.Cu) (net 10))
 (segment (start 128.9 77.96) (end 128.899999 77.13) (width 0.5) (layer F.Cu) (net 11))
 (segment (start 130.83 81.81) (end 130.83 83.59) (width 0.5) (layer F.Cu) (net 14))
 (segment (start 128.9 79.88) (end 130.83 81.81) (width 0.5) (layer F.Cu) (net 14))
 (segment (start 128.9 79.86) (end 128.9 79.88) (width 0.5) (layer F.Cu) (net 14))
 (segment (start 134.59 78.49) (end 134.45 78.35) (width 0.25) (layer F.Cu) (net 9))
 (segment (start 134.59 79.344999) (end 134.59 78.49) (width 0.25) (layer F.Cu) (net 9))
 (segment (start 135.09 80.495) (end 135.09 81.39) (width 0.25) (layer F.Cu) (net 6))
 (segment (start 135.1 83.53) (end 135.1 81.46) (width 0.5) (layer F.Cu) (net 6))
 (segment (start 135.395 83.825) (end 135.1 83.53) (width 0.5) (layer F.Cu) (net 6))
 (segment (start 137.935 83.825) (end 135.395 83.825) (width 0.5) (layer F.Cu) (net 6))
 (segment (start 136.385 80.495) (end 136.46 80.42) (width 0.5) (layer F.Cu) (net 2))
 (segment (start 135.71 80.5) (end 136.505 80.5) (width 0.5) (layer F.Cu) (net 2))
 (segment (start 136.555 80.515) (end 137.935 80.515) (width 0.5) (layer F.Cu) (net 2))
 (segment (start 136.46 80.42) (end 136.555 80.515) (width 0.5) (layer F.Cu) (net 2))
 (segment (start 140.805 80.515) (end 140.804999 78.565) (width 0.5) (layer F.Cu) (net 5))
 (segment (start 140.805 83.825) (end 140.805 81.875) (width 0.5) (layer F.Cu) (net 5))
 (segment (start 140.805 80.515) (end 140.805 81.875) (width 0.5) (layer F.Cu) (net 5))
 (segment (start 140.58001 82.30001) (end 140.805 82.525) (width 0.5) (layer F.Cu) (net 5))
 (segment (start 140.58001 80.201468) (end 140.58001 82.30001) (width 0.5) (layer F.Cu) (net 5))
 (segment (start 140.805 80.426458) (end 140.58001 80.201468) (width 0.5) (layer F.Cu) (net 5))
 (segment (start 140.805 80.515) (end 140.805 80.426458) (width 0.5) (layer F.Cu) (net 5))
 (segment (start 140.47 80.515) (end 140.47 81.875) (width 0.5) (layer F.Cu) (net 5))
 (segment (start 125.34 78.91) (end 125.33 78.92) (width 0.5) (layer F.Cu) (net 1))
 (segment (start 126.7 78.910001) (end 125.34 78.91) (width 0.5) (layer F.Cu) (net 1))
 (segment (start 137.935 83.175) (end 137.934999 81.875) (width 0.5) (layer F.Cu) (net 1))
 (via (at 136.07 81.92) (size 0.4) (drill 0.3) (layers F.Cu B.Cu) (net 1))
 (via (at 136.07 82.66) (size 0.4) (drill 0.3) (layers F.Cu B.Cu) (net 1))
 (via (at 136.82 81.92) (size 0.4) (drill 0.3) (layers F.Cu B.Cu) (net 1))
 (via (at 136.82 82.66) (size 0.4) (drill 0.3) (layers F.Cu B.Cu) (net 1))
 (via (at 124.44 84.7) (size 0.4) (drill 0.3) (layers F.Cu B.Cu) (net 1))
 (via (at 124.44 83.96) (size 0.4) (drill 0.3) (layers F.Cu B.Cu) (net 1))
 (via (at 125.25 84.7) (size 0.4) (drill 0.3) (layers F.Cu B.Cu) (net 1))
 (via (at 126 83.96) (size 0.4) (drill 0.3) (layers F.Cu B.Cu) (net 1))
 (via (at 126 84.7) (size 0.4) (drill 0.3) (layers F.Cu B.Cu) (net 1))
 (via (at 125.25 83.96) (size 0.4) (drill 0.3) (layers F.Cu B.Cu) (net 1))
 (via (at 127.85 84.7) (size 0.4) (drill 0.3) (layers F.Cu B.Cu) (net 1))
 (via (at 127.1 84.7) (size 0.4) (drill 0.3) (layers F.Cu B.Cu) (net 1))
 (via (at 127.85 83.96) (size 0.4) (drill 0.3) (layers F.Cu B.Cu) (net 1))
 (via (at 127.1 83.96) (size 0.4) (drill 0.3) (layers F.Cu B.Cu) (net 1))
 (via (at 126 83.23) (size 0.4) (drill 0.3) (layers F.Cu B.Cu) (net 1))
 (via (at 124.44 83.23) (size 0.4) (drill 0.3) (layers F.Cu B.Cu) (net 1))
 (via (at 125.25 83.23) (size 0.4) (drill 0.3) (layers F.Cu B.Cu) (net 1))
 (via (at 127.85 83.23) (size 0.4) (drill 0.3) (layers F.Cu B.Cu) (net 1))
 (via (at 127.1 83.23) (size 0.4) (drill 0.3) (layers F.Cu B.Cu) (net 1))
 (via (at 125.32 79.809999) (size 0.4) (drill 0.3) (layers F.Cu B.Cu) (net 1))
 (via (at 124.57 79.81) (size 0.4) (drill 0.3) (layers F.Cu B.Cu) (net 1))
 (via (at 124.18 76.87) (size 0.4) (drill 0.3) (layers F.Cu B.Cu) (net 1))
 (via (at 124.93 76.869999) (size 0.4) (drill 0.3) (layers F.Cu B.Cu) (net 1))
 (via (at 124.93 76.099999) (size 0.4) (drill 0.3) (layers F.Cu B.Cu) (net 1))
 (via (at 124.18 76.1) (size 0.4) (drill 0.3) (layers F.Cu B.Cu) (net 1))
 (via (at 126.51 76.869999) (size 0.4) (drill 0.3) (layers F.Cu B.Cu) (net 1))
 (via (at 125.76 76.1) (size 0.4) (drill 0.3) (layers F.Cu B.Cu) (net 1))
 (via (at 125.76 76.87) (size 0.4) (drill 0.3) (layers F.Cu B.Cu) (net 1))
 (via (at 126.51 76.099999) (size 0.4) (drill 0.3) (layers F.Cu B.Cu) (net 1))
 (via (at 132.32 80.139999) (size 0.4) (drill 0.3) (layers F.Cu B.Cu) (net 1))
 (via (at 131.57 80.91) (size 0.4) (drill 0.3) (layers F.Cu B.Cu) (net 1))
 (via (at 132.32 80.909999) (size 0.4) (drill 0.3) (layers F.Cu B.Cu) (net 1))
 (via (at 131.57 80.14) (size 0.4) (drill 0.3) (layers F.Cu B.Cu) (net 1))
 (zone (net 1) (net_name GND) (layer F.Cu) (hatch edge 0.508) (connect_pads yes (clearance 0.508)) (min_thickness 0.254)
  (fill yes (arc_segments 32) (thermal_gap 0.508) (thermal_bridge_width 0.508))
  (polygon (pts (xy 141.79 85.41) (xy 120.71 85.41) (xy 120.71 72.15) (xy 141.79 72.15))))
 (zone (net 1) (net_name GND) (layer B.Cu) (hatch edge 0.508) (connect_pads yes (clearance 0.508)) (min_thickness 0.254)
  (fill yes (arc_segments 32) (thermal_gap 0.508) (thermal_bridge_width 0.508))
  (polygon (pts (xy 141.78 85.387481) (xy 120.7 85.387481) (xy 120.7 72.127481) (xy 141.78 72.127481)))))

